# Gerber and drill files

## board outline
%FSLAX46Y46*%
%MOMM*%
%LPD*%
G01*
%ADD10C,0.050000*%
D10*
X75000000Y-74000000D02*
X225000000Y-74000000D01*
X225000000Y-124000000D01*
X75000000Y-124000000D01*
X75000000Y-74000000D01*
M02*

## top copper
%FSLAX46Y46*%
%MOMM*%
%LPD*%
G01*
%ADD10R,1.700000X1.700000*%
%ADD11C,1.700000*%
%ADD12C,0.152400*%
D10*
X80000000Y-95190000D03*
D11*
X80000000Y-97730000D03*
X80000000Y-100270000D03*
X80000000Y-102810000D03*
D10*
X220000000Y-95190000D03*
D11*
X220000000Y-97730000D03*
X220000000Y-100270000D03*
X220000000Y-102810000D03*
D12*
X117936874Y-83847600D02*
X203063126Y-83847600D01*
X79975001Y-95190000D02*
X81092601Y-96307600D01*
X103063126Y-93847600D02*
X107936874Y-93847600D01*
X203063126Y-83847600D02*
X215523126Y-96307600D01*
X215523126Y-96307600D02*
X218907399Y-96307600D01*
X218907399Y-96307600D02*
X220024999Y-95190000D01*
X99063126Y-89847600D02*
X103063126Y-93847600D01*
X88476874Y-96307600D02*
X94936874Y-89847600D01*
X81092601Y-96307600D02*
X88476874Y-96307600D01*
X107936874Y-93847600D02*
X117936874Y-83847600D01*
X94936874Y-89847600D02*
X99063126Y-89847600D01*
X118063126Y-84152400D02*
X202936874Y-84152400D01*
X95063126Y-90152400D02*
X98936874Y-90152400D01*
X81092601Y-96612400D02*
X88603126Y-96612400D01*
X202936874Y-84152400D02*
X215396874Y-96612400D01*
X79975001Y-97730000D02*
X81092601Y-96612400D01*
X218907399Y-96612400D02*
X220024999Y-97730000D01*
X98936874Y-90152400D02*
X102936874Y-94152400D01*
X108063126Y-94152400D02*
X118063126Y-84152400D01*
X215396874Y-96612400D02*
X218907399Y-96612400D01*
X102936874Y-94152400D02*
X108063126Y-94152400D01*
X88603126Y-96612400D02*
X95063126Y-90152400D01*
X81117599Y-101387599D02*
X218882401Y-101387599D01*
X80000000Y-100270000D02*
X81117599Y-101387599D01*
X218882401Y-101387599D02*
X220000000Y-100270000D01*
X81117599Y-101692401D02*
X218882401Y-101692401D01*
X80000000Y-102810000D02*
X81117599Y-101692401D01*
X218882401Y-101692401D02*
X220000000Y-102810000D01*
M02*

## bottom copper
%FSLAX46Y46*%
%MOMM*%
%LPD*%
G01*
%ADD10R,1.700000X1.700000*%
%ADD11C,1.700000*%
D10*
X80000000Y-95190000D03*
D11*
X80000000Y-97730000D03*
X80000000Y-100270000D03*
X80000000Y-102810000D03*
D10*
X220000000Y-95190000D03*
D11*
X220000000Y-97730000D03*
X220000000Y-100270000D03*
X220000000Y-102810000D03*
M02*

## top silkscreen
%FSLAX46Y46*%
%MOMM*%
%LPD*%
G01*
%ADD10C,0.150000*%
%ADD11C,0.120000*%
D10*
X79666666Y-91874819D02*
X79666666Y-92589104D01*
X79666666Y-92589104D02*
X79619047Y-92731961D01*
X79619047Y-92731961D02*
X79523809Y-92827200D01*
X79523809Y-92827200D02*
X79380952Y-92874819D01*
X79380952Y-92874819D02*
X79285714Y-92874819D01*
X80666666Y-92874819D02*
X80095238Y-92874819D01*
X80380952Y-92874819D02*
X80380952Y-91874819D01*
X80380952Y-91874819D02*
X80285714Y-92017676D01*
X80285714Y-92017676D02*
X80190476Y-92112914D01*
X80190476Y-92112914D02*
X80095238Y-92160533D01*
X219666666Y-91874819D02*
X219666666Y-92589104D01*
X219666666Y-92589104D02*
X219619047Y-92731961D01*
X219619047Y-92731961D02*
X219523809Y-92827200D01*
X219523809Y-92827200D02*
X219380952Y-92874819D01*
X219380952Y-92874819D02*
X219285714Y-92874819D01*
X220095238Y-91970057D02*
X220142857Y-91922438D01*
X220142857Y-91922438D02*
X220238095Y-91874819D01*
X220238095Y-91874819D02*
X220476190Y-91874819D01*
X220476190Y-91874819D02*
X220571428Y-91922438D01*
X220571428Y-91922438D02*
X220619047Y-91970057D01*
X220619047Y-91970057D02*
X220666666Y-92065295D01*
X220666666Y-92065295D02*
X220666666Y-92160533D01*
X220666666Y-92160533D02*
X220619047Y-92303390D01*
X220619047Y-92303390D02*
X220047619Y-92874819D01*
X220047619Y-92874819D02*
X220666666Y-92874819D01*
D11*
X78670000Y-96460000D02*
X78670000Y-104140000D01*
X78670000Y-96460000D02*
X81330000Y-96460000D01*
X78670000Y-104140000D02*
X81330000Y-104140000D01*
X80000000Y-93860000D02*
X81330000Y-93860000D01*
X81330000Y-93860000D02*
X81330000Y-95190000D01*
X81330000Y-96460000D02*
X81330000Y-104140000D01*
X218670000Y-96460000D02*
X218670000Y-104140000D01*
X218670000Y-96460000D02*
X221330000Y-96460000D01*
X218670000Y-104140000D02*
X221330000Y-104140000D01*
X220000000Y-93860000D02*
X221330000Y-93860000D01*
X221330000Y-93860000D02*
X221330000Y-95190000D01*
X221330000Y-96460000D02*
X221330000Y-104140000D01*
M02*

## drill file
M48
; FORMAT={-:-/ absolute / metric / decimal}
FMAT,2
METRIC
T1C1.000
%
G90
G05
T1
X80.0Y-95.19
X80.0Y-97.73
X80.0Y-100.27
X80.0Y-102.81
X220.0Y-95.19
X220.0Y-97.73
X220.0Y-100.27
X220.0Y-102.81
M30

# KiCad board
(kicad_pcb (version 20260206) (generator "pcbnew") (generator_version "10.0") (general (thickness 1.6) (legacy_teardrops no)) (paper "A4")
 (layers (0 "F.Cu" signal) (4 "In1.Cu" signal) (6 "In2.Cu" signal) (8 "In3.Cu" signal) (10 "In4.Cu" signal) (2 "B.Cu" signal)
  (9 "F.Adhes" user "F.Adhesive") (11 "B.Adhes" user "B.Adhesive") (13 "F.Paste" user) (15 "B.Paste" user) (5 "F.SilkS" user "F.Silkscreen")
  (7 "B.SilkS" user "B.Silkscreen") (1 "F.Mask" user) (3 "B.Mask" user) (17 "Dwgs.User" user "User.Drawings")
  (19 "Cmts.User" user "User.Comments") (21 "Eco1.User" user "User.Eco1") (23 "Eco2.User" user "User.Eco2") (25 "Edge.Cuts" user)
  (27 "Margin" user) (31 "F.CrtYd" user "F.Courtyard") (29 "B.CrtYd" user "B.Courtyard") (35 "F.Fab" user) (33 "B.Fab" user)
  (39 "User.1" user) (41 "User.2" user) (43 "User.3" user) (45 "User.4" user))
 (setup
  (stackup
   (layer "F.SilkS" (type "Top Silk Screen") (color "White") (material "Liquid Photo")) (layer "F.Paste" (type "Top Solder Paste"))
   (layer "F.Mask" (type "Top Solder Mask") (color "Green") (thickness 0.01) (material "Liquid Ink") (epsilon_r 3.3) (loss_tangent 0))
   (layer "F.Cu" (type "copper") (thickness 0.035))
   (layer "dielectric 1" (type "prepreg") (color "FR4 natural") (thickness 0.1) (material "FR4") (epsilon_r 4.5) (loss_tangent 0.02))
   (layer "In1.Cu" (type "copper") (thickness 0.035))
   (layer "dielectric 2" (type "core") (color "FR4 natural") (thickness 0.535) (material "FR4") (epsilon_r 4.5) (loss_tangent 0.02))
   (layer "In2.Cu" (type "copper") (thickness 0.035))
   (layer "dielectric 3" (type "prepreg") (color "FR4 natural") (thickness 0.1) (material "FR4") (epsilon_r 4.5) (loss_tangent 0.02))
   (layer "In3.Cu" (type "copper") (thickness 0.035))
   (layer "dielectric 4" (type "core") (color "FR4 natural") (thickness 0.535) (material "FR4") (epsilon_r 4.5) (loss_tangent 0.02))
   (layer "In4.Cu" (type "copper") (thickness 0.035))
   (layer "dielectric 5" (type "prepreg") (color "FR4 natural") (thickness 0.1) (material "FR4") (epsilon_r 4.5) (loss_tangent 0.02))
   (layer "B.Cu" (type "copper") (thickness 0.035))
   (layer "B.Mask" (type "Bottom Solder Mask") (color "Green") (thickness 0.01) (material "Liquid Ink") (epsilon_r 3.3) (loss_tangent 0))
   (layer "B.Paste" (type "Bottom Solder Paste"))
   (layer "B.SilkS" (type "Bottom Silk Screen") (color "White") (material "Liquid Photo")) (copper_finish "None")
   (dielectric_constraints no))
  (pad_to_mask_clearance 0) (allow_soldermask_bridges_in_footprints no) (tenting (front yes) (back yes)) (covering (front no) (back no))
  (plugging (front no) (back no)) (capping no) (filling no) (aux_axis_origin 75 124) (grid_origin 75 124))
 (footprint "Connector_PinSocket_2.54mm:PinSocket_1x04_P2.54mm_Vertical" (layer "F.Cu") (at 80 95.19)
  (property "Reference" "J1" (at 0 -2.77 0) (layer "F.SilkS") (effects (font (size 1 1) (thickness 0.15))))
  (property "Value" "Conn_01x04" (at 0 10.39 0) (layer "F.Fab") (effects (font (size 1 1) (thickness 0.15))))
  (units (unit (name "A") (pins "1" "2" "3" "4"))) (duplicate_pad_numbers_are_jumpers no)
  (fp_line (start -1.33 1.27) (end -1.33 8.95) (stroke (width 0.12) (type solid)) (layer "F.SilkS"))
  (fp_line (start -1.33 1.27) (end 1.33 1.27) (stroke (width 0.12) (type solid)) (layer "F.SilkS"))
  (fp_line (start -1.33 8.95) (end 1.33 8.95) (stroke (width 0.12) (type solid)) (layer "F.SilkS"))
  (fp_line (start 0 -1.33) (end 1.33 -1.33) (stroke (width 0.12) (type solid)) (layer "F.SilkS"))
  (fp_line (start 1.33 -1.33) (end 1.33 0) (stroke (width 0.12) (type solid)) (layer "F.SilkS"))
  (fp_line (start 1.33 1.27) (end 1.33 8.95) (stroke (width 0.12) (type solid)) (layer "F.SilkS"))
  (pad "1" thru_hole rect (at 0 0) (size 1.7 1.7) (drill 1) (layers "*.Cu" "*.Mask") (remove_unused_layers no) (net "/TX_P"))
  (pad "2" thru_hole circle (at 0 2.54) (size 1.7 1.7) (drill 1) (layers "*.Cu" "*.Mask") (remove_unused_layers no) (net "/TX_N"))
  (pad "3" thru_hole circle (at 0 5.08) (size 1.7 1.7) (drill 1) (layers "*.Cu" "*.Mask") (remove_unused_layers no) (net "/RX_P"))
  (pad "4" thru_hole circle (at 0 7.62) (size 1.7 1.7) (drill 1) (layers "*.Cu" "*.Mask") (remove_unused_layers no) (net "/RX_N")))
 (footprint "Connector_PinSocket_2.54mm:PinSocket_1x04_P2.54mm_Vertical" (layer "F.Cu") (at 220 95.19)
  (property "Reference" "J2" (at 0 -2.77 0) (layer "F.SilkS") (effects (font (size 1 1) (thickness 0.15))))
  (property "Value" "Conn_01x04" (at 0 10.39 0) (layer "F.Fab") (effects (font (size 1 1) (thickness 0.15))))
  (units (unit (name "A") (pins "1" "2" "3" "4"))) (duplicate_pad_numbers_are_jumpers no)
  (fp_line (start -1.33 1.27) (end -1.33 8.95) (stroke (width 0.12) (type solid)) (layer "F.SilkS"))
  (fp_line (start -1.33 1.27) (end 1.33 1.27) (stroke (width 0.12) (type solid)) (layer "F.SilkS"))
  (fp_line (start -1.33 8.95) (end 1.33 8.95) (stroke (width 0.12) (type solid)) (layer "F.SilkS"))
  (fp_line (start 0 -1.33) (end 1.33 -1.33) (stroke (width 0.12) (type solid)) (layer "F.SilkS"))
  (fp_line (start 1.33 -1.33) (end 1.33 0) (stroke (width 0.12) (type solid)) (layer "F.SilkS"))
  (fp_line (start 1.33 1.27) (end 1.33 8.95) (stroke (width 0.12) (type solid)) (layer "F.SilkS"))
  (pad "1" thru_hole rect (at 0 0) (size 1.7 1.7) (drill 1) (layers "*.Cu" "*.Mask") (remove_unused_layers no) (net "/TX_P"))
  (pad "2" thru_hole circle (at 0 2.54) (size 1.7 1.7) (drill 1) (layers "*.Cu" "*.Mask") (remove_unused_layers no) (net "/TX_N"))
  (pad "3" thru_hole circle (at 0 5.08) (size 1.7 1.7) (drill 1) (layers "*.Cu" "*.Mask") (remove_unused_layers no) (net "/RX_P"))
  (pad "4" thru_hole circle (at 0 7.62) (size 1.7 1.7) (drill 1) (layers "*.Cu" "*.Mask") (remove_unused_layers no) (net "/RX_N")))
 (gr_rect (start 75 74) (end 225 124) (stroke (width 0.05) (type solid)) (fill no) (layer "Edge.Cuts"))
 (segment (start 117.936874 83.8476) (end 203.063126 83.8476) (width 0.1524) (layer "F.Cu") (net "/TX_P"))
 (segment (start 79.975001 95.19) (end 81.092601 96.3076) (width 0.1524) (layer "F.Cu") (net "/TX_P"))
 (segment (start 103.063126 93.8476) (end 107.936874 93.8476) (width 0.1524) (layer "F.Cu") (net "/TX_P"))
 (segment (start 203.063126 83.8476) (end 215.523126 96.3076) (width 0.1524) (layer "F.Cu") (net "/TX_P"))
 (segment (start 215.523126 96.3076) (end 218.907399 96.3076) (width 0.1524) (layer "F.Cu") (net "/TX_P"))
 (segment (start 218.907399 96.3076) (end 220.024999 95.19) (width 0.1524) (layer "F.Cu") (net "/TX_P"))
 (segment (start 99.063126 89.8476) (end 103.063126 93.8476) (width 0.1524) (layer "F.Cu") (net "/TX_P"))
 (segment (start 88.476874 96.3076) (end 94.936874 89.8476) (width 0.1524) (layer "F.Cu") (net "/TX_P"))
 (segment (start 81.092601 96.3076) (end 88.476874 96.3076) (width 0.1524) (layer "F.Cu") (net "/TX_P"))
 (segment (start 107.936874 93.8476) (end 117.936874 83.8476) (width 0.1524) (layer "F.Cu") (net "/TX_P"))
 (segment (start 94.936874 89.8476) (end 99.063126 89.8476) (width 0.1524) (layer "F.Cu") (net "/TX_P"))
 (segment (start 118.063126 84.1524) (end 202.936874 84.1524) (width 0.1524) (layer "F.Cu") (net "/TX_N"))
 (segment (start 95.063126 90.1524) (end 98.936874 90.1524) (width 0.1524) (layer "F.Cu") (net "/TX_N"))
 (segment (start 81.092601 96.6124) (end 88.603126 96.6124) (width 0.1524) (layer "F.Cu") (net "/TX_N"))
 (segment (start 202.936874 84.1524) (end 215.396874 96.6124) (width 0.1524) (layer "F.Cu") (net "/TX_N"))
 (segment (start 79.975001 97.73) (end 81.092601 96.6124) (width 0.1524) (layer "F.Cu") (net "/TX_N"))
 (segment (start 218.907399 96.6124) (end 220.024999 97.73) (width 0.1524) (layer "F.Cu") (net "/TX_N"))
 (segment (start 98.936874 90.1524) (end 102.936874 94.1524) (width 0.1524) (layer "F.Cu") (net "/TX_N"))
 (segment (start 108.063126 94.1524) (end 118.063126 84.1524) (width 0.1524) (layer "F.Cu") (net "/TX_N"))
 (segment (start 215.396874 96.6124) (end 218.907399 96.6124) (width 0.1524) (layer "F.Cu") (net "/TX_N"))
 (segment (start 102.936874 94.1524) (end 108.063126 94.1524) (width 0.1524) (layer "F.Cu") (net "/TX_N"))
 (segment (start 88.603126 96.6124) (end 95.063126 90.1524) (width 0.1524) (layer "F.Cu") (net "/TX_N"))
 (segment (start 81.117599 101.387599) (end 218.882401 101.387599) (width 0.1524) (layer "F.Cu") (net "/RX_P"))
 (segment (start 80 100.27) (end 81.117599 101.387599) (width 0.1524) (layer "F.Cu") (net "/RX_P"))
 (segment (start 218.882401 101.387599) (end 220 100.27) (width 0.1524) (layer "F.Cu") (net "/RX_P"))
 (segment (start 81.117599 101.692401) (end 218.882401 101.692401) (width 0.1524) (layer "F.Cu") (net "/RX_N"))
 (segment (start 80 102.81) (end 81.117599 101.692401) (width 0.1524) (layer "F.Cu") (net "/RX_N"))
 (segment (start 218.882401 101.692401) (end 220 102.81) (width 0.1524) (layer "F.Cu") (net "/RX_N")))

